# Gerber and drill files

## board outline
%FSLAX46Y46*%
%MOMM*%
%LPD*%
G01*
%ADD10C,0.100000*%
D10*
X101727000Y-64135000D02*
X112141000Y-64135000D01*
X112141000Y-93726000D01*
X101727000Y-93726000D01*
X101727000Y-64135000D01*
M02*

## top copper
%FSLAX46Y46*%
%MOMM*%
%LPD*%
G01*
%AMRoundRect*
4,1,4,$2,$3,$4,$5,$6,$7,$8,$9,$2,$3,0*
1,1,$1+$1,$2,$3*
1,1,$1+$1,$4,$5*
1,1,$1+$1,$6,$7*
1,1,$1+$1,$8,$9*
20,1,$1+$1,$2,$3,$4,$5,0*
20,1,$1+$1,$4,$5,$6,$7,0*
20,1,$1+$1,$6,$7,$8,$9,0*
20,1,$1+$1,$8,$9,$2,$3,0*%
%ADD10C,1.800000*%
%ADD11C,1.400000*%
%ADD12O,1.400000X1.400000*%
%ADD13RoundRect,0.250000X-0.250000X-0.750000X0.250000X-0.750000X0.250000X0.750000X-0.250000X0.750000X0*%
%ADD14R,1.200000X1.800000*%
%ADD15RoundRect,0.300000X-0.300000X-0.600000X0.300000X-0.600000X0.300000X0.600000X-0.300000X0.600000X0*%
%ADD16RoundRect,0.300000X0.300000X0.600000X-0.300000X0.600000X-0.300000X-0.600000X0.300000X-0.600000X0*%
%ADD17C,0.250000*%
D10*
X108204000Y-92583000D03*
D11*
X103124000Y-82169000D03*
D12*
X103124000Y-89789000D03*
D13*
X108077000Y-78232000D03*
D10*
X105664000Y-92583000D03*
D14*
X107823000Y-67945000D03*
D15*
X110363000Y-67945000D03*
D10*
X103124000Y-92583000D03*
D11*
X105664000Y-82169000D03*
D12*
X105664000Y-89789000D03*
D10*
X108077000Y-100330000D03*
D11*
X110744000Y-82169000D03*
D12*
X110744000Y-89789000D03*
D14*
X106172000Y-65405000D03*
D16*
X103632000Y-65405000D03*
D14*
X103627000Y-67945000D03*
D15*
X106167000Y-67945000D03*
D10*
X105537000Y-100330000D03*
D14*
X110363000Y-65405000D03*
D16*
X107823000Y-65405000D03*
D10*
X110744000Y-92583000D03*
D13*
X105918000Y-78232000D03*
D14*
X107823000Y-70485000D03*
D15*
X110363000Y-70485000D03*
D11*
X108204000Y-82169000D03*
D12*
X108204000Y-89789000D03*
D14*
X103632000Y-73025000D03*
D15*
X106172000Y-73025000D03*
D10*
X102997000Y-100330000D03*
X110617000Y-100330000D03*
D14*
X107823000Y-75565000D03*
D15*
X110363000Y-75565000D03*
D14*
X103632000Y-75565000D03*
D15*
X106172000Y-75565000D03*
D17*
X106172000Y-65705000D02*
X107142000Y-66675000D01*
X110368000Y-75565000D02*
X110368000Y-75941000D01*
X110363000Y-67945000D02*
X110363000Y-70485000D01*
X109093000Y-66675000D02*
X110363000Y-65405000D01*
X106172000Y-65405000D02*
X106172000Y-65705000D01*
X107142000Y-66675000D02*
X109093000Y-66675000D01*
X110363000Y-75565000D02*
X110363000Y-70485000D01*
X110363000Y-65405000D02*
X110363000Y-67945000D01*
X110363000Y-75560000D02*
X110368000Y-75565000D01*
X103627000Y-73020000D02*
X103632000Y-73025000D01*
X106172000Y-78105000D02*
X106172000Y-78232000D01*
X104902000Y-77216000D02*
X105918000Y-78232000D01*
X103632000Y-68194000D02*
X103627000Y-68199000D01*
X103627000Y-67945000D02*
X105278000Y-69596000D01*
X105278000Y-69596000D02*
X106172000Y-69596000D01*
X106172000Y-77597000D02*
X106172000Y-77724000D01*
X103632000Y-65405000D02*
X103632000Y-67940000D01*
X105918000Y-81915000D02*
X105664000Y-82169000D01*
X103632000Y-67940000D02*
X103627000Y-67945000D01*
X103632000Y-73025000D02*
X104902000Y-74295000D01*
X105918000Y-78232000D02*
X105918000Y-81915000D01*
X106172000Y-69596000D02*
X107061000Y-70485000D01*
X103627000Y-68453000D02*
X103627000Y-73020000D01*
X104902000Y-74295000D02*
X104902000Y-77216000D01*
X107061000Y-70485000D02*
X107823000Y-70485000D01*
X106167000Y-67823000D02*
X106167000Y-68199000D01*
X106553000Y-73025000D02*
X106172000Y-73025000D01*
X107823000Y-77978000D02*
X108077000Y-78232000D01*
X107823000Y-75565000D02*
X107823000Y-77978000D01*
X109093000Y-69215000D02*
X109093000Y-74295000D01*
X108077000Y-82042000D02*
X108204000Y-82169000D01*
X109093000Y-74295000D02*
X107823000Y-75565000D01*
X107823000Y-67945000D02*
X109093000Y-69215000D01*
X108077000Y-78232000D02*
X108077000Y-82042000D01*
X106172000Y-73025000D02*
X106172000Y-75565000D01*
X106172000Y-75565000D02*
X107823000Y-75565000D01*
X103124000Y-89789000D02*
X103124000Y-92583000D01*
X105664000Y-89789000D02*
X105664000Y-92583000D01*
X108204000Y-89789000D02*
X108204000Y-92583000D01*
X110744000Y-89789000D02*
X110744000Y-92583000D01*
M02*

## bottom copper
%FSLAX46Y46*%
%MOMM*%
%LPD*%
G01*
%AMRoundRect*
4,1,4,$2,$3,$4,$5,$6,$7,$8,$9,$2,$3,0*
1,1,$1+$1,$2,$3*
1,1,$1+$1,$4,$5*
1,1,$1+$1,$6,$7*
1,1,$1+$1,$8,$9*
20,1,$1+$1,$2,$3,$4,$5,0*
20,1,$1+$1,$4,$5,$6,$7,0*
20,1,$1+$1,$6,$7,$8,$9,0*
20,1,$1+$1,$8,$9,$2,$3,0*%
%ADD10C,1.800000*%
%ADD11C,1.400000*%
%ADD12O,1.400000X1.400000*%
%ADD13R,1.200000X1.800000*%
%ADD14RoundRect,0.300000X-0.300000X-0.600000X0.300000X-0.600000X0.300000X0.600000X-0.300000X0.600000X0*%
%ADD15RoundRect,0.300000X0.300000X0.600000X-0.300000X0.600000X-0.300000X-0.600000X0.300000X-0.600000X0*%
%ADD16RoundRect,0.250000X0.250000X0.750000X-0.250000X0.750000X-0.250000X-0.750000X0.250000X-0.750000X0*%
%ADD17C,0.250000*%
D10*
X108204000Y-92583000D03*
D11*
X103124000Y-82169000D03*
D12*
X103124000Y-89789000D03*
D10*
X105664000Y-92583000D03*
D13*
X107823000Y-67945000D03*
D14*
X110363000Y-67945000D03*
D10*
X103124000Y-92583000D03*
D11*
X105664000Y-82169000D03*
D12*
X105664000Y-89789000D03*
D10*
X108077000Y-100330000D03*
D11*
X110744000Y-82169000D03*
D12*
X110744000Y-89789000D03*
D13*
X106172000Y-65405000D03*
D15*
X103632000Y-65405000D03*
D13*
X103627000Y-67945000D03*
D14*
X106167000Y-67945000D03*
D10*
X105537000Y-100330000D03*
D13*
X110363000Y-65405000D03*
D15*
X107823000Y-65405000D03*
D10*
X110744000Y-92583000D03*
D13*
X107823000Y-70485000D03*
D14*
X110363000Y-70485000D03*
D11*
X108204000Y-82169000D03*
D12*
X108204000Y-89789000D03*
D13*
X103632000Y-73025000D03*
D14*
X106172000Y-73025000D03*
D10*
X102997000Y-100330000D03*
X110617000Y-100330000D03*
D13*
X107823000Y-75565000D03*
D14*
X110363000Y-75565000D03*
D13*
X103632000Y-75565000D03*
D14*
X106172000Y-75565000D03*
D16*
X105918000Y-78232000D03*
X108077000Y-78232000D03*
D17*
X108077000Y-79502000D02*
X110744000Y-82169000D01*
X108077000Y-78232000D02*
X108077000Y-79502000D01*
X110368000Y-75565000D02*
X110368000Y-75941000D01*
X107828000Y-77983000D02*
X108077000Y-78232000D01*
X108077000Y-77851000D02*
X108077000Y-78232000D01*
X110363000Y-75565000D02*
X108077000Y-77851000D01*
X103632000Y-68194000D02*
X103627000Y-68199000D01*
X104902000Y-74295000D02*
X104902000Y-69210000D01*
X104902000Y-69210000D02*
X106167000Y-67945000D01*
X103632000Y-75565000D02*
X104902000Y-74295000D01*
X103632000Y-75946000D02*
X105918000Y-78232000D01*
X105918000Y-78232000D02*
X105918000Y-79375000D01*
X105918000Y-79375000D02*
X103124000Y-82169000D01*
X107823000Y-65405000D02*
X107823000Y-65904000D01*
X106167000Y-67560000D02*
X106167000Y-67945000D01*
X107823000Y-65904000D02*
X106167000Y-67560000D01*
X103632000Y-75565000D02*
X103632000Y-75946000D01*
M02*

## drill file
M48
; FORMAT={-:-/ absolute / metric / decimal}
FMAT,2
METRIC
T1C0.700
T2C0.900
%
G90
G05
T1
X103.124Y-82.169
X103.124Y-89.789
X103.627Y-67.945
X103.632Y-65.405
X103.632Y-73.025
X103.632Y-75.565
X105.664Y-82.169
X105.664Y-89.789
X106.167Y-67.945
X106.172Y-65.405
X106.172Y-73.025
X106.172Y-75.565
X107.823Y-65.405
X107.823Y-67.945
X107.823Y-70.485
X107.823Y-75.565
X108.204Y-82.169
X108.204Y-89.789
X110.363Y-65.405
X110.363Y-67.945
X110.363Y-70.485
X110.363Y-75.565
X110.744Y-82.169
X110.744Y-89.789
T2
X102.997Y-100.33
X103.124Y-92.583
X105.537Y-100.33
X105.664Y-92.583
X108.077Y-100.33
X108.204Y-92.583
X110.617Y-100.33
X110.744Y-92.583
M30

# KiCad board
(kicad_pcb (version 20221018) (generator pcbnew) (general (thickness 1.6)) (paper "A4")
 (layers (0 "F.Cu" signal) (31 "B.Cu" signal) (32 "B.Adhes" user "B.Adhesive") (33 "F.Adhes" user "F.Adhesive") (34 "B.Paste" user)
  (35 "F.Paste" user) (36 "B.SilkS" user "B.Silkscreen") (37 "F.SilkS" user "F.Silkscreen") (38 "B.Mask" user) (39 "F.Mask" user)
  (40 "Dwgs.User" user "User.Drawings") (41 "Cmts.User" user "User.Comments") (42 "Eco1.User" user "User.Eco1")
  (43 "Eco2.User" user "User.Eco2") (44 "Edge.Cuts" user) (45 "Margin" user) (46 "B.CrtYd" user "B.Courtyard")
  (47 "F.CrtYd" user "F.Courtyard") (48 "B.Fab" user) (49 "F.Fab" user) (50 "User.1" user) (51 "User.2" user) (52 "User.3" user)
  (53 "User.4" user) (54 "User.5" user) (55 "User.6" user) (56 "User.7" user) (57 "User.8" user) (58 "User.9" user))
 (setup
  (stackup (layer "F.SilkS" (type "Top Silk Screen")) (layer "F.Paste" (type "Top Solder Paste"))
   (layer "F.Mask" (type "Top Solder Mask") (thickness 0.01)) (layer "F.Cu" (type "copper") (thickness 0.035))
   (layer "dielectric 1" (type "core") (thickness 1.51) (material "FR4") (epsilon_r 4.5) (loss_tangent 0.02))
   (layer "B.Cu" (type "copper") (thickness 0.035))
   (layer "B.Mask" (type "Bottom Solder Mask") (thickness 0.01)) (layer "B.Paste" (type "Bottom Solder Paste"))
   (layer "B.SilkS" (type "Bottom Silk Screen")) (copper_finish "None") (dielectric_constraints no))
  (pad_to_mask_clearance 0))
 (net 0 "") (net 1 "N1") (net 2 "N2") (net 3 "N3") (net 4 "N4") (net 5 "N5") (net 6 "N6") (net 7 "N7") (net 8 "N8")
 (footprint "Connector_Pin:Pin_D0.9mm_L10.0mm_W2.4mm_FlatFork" (layer "F.Cu") (at 108.204 92.583)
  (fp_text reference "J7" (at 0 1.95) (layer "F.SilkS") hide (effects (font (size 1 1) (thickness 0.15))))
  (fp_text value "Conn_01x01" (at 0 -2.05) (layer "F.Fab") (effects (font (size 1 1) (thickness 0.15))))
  (pad "1" thru_hole circle (at 0 0) (size 1.8 1.8) (drill 0.9) (layers "*.Cu" "*.Mask") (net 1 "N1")))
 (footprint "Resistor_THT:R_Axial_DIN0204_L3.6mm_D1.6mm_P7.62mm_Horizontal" (layer "F.Cu") (at 103.124 82.169 -90)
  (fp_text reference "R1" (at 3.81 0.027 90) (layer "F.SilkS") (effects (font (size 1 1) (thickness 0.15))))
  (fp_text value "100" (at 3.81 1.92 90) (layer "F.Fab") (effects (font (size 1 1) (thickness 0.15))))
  (pad "1" thru_hole circle (at 0 0 270) (size 1.4 1.4) (drill 0.7) (layers "*.Cu" "*.Mask") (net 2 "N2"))
  (pad "2" thru_hole oval (at 7.62 0 270) (size 1.4 1.4) (drill 0.7) (layers "*.Cu" "*.Mask") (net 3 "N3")))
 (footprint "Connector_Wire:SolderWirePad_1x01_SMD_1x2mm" (layer "F.Cu") (at 108.077 78.232)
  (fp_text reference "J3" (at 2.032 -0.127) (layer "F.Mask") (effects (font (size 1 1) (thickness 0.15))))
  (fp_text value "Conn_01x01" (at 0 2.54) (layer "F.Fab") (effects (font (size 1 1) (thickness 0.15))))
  (pad "1" smd roundrect (at 0 0) (size 1 2) (layers "F.Cu" "F.Paste" "F.Mask") (roundrect_rratio 0.25) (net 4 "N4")))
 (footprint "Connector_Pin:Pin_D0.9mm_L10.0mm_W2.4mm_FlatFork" (layer "F.Cu") (at 105.664 92.583)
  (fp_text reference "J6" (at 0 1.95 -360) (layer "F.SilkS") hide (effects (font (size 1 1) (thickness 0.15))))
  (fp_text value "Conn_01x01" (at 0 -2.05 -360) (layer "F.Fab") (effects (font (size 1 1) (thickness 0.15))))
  (pad "1" thru_hole circle (at 0 0) (size 1.8 1.8) (drill 0.9) (layers "*.Cu" "*.Mask") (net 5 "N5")))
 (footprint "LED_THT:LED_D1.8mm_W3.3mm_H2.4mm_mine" (layer "F.Cu") (at 107.823 67.945)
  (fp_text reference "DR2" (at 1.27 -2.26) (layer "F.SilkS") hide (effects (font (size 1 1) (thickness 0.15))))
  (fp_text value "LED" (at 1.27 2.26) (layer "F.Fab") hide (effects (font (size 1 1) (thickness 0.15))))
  (pad "1" thru_hole rect (at 0 0) (size 1.2 1.8) (drill 0.7) (layers "*.Cu" "*.Mask") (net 4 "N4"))
  (pad "2" thru_hole roundrect (at 2.54 0) (size 1.2 1.8) (drill 0.7) (layers "*.Cu" "*.Mask") (roundrect_rratio 0.25) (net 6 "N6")))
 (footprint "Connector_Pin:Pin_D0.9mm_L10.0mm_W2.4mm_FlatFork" (layer "F.Cu") (at 103.124 92.583)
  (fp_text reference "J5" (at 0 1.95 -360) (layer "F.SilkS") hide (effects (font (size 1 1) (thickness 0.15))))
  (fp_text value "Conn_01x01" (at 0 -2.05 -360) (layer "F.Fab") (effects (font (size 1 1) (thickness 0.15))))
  (pad "1" thru_hole circle (at 0 0) (size 1.8 1.8) (drill 0.9) (layers "*.Cu" "*.Mask") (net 3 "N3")))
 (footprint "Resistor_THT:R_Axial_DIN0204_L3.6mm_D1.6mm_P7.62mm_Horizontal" (layer "F.Cu") (at 105.664 82.169 -90)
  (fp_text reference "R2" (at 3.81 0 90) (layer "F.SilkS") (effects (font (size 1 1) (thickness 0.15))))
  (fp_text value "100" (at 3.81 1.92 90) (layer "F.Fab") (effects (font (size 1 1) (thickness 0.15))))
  (pad "1" thru_hole circle (at 0 0 270) (size 1.4 1.4) (drill 0.7) (layers "*.Cu" "*.Mask") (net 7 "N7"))
  (pad "2" thru_hole oval (at 7.62 0 270) (size 1.4 1.4) (drill 0.7) (layers "*.Cu" "*.Mask") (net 5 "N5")))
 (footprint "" (layer "F.Cu") (at 108.077 100.33)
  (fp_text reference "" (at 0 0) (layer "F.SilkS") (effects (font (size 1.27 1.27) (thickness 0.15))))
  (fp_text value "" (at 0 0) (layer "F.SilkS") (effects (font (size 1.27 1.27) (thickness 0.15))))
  (pad "1" thru_hole circle (at 0 0) (size 1.8 1.8) (drill 0.9) (layers "*.Cu" "*.Mask")))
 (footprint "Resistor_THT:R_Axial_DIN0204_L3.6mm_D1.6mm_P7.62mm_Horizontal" (layer "F.Cu") (at 110.744 82.169 -90)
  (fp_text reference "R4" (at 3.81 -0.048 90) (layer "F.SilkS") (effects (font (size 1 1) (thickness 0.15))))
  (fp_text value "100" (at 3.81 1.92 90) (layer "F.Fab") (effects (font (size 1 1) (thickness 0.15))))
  (pad "1" thru_hole circle (at 0 0 270) (size 1.4 1.4) (drill 0.7) (layers "*.Cu" "*.Mask") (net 6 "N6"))
  (pad "2" thru_hole oval (at 7.62 0 270) (size 1.4 1.4) (drill 0.7) (layers "*.Cu" "*.Mask") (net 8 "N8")))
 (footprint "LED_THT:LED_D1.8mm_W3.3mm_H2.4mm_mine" (layer "F.Cu") (at 106.172 65.405 180)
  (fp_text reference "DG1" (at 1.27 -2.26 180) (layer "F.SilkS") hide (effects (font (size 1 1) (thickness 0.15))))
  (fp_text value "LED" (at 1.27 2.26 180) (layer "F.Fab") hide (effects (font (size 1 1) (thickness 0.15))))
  (pad "1" thru_hole rect (at 0 0 180) (size 1.2 1.8) (drill 0.7) (layers "*.Cu" "*.Mask") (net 6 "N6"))
  (pad "2" thru_hole roundrect (at 2.54 0 180) (size 1.2 1.8) (drill 0.7) (layers "*.Cu" "*.Mask") (roundrect_rratio 0.25) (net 7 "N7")))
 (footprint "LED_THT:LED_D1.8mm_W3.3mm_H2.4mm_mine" (layer "F.Cu") (at 103.627 67.945)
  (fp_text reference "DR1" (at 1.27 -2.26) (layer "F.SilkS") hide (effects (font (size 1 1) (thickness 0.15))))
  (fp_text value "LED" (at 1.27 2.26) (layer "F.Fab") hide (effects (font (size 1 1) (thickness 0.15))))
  (pad "1" thru_hole rect (at 0 0) (size 1.2 1.8) (drill 0.7) (layers "*.Cu" "*.Mask") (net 7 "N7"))
  (pad "2" thru_hole roundrect (at 2.54 0) (size 1.2 1.8) (drill 0.7) (layers "*.Cu" "*.Mask") (roundrect_rratio 0.25) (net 2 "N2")))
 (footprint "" (layer "F.Cu") (at 105.537 100.33)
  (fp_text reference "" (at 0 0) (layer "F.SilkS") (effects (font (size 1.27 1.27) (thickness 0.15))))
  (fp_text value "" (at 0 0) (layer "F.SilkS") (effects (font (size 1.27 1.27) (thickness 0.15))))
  (pad "1" thru_hole circle (at 0 0) (size 1.8 1.8) (drill 0.9) (layers "*.Cu" "*.Mask")))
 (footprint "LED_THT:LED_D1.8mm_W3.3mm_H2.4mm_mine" (layer "F.Cu") (at 110.363 65.405 180)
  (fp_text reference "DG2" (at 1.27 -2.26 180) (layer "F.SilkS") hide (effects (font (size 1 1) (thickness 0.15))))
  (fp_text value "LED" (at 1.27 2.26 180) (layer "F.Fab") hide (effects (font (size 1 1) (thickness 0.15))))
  (pad "1" thru_hole rect (at 0 0 180) (size 1.2 1.8) (drill 0.7) (layers "*.Cu" "*.Mask") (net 6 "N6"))
  (pad "2" thru_hole roundrect (at 2.54 0 180) (size 1.2 1.8) (drill 0.7) (layers "*.Cu" "*.Mask") (roundrect_rratio 0.25) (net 2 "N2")))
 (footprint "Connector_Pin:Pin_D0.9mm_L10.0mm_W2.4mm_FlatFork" (layer "F.Cu") (at 110.744 92.583)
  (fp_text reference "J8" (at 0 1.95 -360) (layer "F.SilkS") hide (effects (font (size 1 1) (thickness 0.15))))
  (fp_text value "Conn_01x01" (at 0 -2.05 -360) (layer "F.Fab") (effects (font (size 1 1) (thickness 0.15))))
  (pad "1" thru_hole circle (at 0 0) (size 1.8 1.8) (drill 0.9) (layers "*.Cu" "*.Mask") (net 8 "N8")))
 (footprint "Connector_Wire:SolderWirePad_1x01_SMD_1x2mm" (layer "F.Cu") (at 105.918 78.232)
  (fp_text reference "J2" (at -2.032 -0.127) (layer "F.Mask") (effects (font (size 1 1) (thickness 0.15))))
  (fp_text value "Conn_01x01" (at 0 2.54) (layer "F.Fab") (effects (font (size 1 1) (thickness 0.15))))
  (pad "1" smd roundrect (at 0 0) (size 1 2) (layers "F.Cu" "F.Paste" "F.Mask") (roundrect_rratio 0.25) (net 7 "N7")))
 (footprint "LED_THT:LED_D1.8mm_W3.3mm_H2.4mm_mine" (layer "F.Cu") (at 107.823 70.485)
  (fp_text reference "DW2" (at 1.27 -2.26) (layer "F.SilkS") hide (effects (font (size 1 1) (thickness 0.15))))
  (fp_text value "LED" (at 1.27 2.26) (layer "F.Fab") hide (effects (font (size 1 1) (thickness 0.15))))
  (pad "1" thru_hole rect (at 0 0) (size 1.2 1.8) (drill 0.7) (layers "*.Cu" "*.Mask") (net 7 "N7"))
  (pad "2" thru_hole roundrect (at 2.54 0) (size 1.2 1.8) (drill 0.7) (layers "*.Cu" "*.Mask") (roundrect_rratio 0.25) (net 6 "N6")))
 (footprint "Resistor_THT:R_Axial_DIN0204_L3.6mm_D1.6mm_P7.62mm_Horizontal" (layer "F.Cu") (at 108.204 82.169 -90)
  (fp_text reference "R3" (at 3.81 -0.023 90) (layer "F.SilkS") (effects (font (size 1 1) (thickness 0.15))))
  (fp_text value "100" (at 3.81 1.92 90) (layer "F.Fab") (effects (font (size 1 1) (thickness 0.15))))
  (pad "1" thru_hole circle (at 0 0 270) (size 1.4 1.4) (drill 0.7) (layers "*.Cu" "*.Mask") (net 4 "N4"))
  (pad "2" thru_hole oval (at 7.62 0 270) (size 1.4 1.4) (drill 0.7) (layers "*.Cu" "*.Mask") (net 1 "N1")))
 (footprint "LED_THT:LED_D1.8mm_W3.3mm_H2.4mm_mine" (layer "F.Cu") (at 103.632 73.025)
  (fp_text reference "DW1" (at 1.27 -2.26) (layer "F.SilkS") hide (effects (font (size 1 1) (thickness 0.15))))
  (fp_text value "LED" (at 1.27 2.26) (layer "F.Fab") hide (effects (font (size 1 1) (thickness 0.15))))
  (pad "1" thru_hole rect (at 0 0) (size 1.2 1.8) (drill 0.7) (layers "*.Cu" "*.Mask") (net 7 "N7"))
  (pad "2" thru_hole roundrect (at 2.54 0) (size 1.2 1.8) (drill 0.7) (layers "*.Cu" "*.Mask") (roundrect_rratio 0.25) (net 4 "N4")))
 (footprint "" (layer "F.Cu") (at 102.997 100.33)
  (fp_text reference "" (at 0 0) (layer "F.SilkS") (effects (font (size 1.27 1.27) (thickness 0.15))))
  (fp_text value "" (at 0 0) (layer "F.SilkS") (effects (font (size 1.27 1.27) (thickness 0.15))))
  (pad "1" thru_hole circle (at 0 0) (size 1.8 1.8) (drill 0.9) (layers "*.Cu" "*.Mask")))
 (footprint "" (layer "F.Cu") (at 110.617 100.33)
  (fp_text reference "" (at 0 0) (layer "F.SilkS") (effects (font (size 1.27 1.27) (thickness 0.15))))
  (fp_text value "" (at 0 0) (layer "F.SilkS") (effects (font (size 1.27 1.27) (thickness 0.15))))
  (pad "1" thru_hole circle (at 0 0) (size 1.8 1.8) (drill 0.9) (layers "*.Cu" "*.Mask")))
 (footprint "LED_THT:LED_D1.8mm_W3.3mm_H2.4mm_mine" (layer "B.Cu") (at 107.823 75.565)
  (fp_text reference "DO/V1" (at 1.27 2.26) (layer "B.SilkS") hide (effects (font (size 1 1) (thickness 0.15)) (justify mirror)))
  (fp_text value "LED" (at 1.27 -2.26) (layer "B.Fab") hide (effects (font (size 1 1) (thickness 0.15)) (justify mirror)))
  (pad "1" thru_hole rect (at 0 0) (size 1.2 1.8) (drill 0.7) (layers "*.Cu" "*.Mask") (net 4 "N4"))
  (pad "2" thru_hole roundrect (at 2.54 0) (size 1.2 1.8) (drill 0.7) (layers "*.Cu" "*.Mask") (roundrect_rratio 0.25) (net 6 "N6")))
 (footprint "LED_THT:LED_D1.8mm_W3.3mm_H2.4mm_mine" (layer "B.Cu") (at 103.632 75.565)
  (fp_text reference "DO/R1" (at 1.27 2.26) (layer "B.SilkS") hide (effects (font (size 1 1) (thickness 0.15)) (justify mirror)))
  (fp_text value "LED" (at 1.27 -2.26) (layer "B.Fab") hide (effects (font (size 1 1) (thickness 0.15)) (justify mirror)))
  (pad "1" thru_hole rect (at 0 0) (size 1.2 1.8) (drill 0.7) (layers "*.Cu" "*.Mask") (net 2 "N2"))
  (pad "2" thru_hole roundrect (at 2.54 0) (size 1.2 1.8) (drill 0.7) (layers "*.Cu" "*.Mask") (roundrect_rratio 0.25) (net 4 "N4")))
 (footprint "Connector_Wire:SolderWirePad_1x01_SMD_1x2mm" (layer "B.Cu") (at 105.918 78.232 180)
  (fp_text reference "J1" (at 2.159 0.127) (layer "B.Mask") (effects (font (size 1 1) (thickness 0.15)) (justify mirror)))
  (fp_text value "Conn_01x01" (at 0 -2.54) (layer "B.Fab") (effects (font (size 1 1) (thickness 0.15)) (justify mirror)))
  (pad "1" smd roundrect (at 0 0 180) (size 1 2) (layers "B.Cu" "B.Paste" "B.Mask") (roundrect_rratio 0.25) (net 2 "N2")))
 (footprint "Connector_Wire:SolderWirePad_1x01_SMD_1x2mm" (layer "B.Cu") (at 108.077 78.232 180)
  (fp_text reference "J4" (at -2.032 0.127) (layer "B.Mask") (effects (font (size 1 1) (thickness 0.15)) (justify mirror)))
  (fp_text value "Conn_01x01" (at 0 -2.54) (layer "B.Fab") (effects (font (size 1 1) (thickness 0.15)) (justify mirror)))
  (pad "1" smd roundrect (at 0 0 180) (size 1 2) (layers "B.Cu" "B.Paste" "B.Mask") (roundrect_rratio 0.25) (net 6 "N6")))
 (gr_rect (start 101.727 64.135) (end 112.141 93.726) (stroke (width 0.1) (type default)) (fill none) (layer "Edge.Cuts"))
 (segment (start 106.172 65.705) (end 107.142 66.675) (width 0.25) (layer "F.Cu") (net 6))
 (segment (start 110.368 75.565) (end 110.368 75.941) (width 0.25) (layer "F.Cu") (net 6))
 (segment (start 110.363 67.945) (end 110.363 70.485) (width 0.25) (layer "F.Cu") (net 6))
 (segment (start 109.093 66.675) (end 110.363 65.405) (width 0.25) (layer "F.Cu") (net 6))
 (segment (start 106.172 65.405) (end 106.172 65.705) (width 0.25) (layer "F.Cu") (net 6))
 (segment (start 107.142 66.675) (end 109.093 66.675) (width 0.25) (layer "F.Cu") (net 6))
 (segment (start 110.363 75.565) (end 110.363 70.485) (width 0.25) (layer "F.Cu") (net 6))
 (segment (start 110.363 65.405) (end 110.363 67.945) (width 0.25) (layer "F.Cu") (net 6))
 (segment (start 110.363 75.56) (end 110.368 75.565) (width 0.25) (layer "F.Cu") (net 6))
 (segment (start 108.077 79.502) (end 110.744 82.169) (width 0.25) (layer "B.Cu") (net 6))
 (segment (start 108.077 78.232) (end 108.077 79.502) (width 0.25) (layer "B.Cu") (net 6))
 (segment (start 110.368 75.565) (end 110.368 75.941) (width 0.25) (layer "B.Cu") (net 6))
 (segment (start 107.828 77.983) (end 108.077 78.232) (width 0.25) (layer "B.Cu") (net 6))
 (segment (start 108.077 77.851) (end 108.077 78.232) (width 0.25) (layer "B.Cu") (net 6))
 (segment (start 110.363 75.565) (end 108.077 77.851) (width 0.25) (layer "B.Cu") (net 6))
 (segment (start 103.627 73.02) (end 103.632 73.025) (width 0.25) (layer "F.Cu") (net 7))
 (segment (start 106.172 78.105) (end 106.172 78.232) (width 0.25) (layer "F.Cu") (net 7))
 (segment (start 104.902 77.216) (end 105.918 78.232) (width 0.25) (layer "F.Cu") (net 7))
 (segment (start 103.632 68.194) (end 103.627 68.199) (width 0.25) (layer "F.Cu") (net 7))
 (segment (start 103.627 67.945) (end 105.278 69.596) (width 0.25) (layer "F.Cu") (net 7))
 (segment (start 105.278 69.596) (end 106.172 69.596) (width 0.25) (layer "F.Cu") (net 7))
 (segment (start 106.172 77.597) (end 106.172 77.724) (width 0.25) (layer "F.Cu") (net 7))
 (segment (start 103.632 65.405) (end 103.632 67.94) (width 0.25) (layer "F.Cu") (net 7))
 (segment (start 105.918 81.915) (end 105.664 82.169) (width 0.25) (layer "F.Cu") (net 7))
 (segment (start 103.632 67.94) (end 103.627 67.945) (width 0.25) (layer "F.Cu") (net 7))
 (segment (start 103.632 73.025) (end 104.902 74.295) (width 0.25) (layer "F.Cu") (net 7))
 (segment (start 105.918 78.232) (end 105.918 81.915) (width 0.25) (layer "F.Cu") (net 7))
 (segment (start 106.172 69.596) (end 107.061 70.485) (width 0.25) (layer "F.Cu") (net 7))
 (segment (start 103.627 68.453) (end 103.627 73.02) (width 0.25) (layer "F.Cu") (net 7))
 (segment (start 104.902 74.295) (end 104.902 77.216) (width 0.25) (layer "F.Cu") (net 7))
 (segment (start 107.061 70.485) (end 107.823 70.485) (width 0.25) (layer "F.Cu") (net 7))
 (segment (start 103.632 68.194) (end 103.627 68.199) (width 0.25) (layer "B.Cu") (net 7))
 (segment (start 106.167 67.823) (end 106.167 68.199) (width 0.25) (layer "F.Cu") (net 2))
 (segment (start 104.902 74.295) (end 104.902 69.21) (width 0.25) (layer "B.Cu") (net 2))
 (segment (start 104.902 69.21) (end 106.167 67.945) (width 0.25) (layer "B.Cu") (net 2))
 (segment (start 103.632 75.565) (end 104.902 74.295) (width 0.25) (layer "B.Cu") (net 2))
 (segment (start 103.632 75.946) (end 105.918 78.232) (width 0.25) (layer "B.Cu") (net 2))
 (segment (start 105.918 78.232) (end 105.918 79.375) (width 0.25) (layer "B.Cu") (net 2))
 (segment (start 105.918 79.375) (end 103.124 82.169) (width 0.25) (layer "B.Cu") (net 2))
 (segment (start 107.823 65.405) (end 107.823 65.904) (width 0.25) (layer "B.Cu") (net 2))
 (segment (start 106.167 67.56) (end 106.167 67.945) (width 0.25) (layer "B.Cu") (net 2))
 (segment (start 107.823 65.904) (end 106.167 67.56) (width 0.25) (layer "B.Cu") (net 2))
 (segment (start 103.632 75.565) (end 103.632 75.946) (width 0.25) (layer "B.Cu") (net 2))
 (segment (start 106.553 73.025) (end 106.172 73.025) (width 0.25) (layer "F.Cu") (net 4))
 (segment (start 107.823 77.978) (end 108.077 78.232) (width 0.25) (layer "F.Cu") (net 4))
 (segment (start 107.823 75.565) (end 107.823 77.978) (width 0.25) (layer "F.Cu") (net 4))
 (segment (start 109.093 69.215) (end 109.093 74.295) (width 0.25) (layer "F.Cu") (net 4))
 (segment (start 108.077 82.042) (end 108.204 82.169) (width 0.25) (layer "F.Cu") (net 4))
 (segment (start 109.093 74.295) (end 107.823 75.565) (width 0.25) (layer "F.Cu") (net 4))
 (segment (start 107.823 67.945) (end 109.093 69.215) (width 0.25) (layer "F.Cu") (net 4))
 (segment (start 108.077 78.232) (end 108.077 82.042) (width 0.25) (layer "F.Cu") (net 4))
 (segment (start 106.172 73.025) (end 106.172 75.565) (width 0.25) (layer "F.Cu") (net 4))
 (segment (start 106.172 75.565) (end 107.823 75.565) (width 0.25) (layer "F.Cu") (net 4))
 (segment (start 103.124 89.789) (end 103.124 92.583) (width 0.25) (layer "F.Cu") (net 3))
 (segment (start 105.664 89.789) (end 105.664 92.583) (width 0.25) (layer "F.Cu") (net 5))
 (segment (start 108.204 89.789) (end 108.204 92.583) (width 0.25) (layer "F.Cu") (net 1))
 (segment (start 110.744 89.789) (end 110.744 92.583) (width 0.25) (layer "F.Cu") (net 8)))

